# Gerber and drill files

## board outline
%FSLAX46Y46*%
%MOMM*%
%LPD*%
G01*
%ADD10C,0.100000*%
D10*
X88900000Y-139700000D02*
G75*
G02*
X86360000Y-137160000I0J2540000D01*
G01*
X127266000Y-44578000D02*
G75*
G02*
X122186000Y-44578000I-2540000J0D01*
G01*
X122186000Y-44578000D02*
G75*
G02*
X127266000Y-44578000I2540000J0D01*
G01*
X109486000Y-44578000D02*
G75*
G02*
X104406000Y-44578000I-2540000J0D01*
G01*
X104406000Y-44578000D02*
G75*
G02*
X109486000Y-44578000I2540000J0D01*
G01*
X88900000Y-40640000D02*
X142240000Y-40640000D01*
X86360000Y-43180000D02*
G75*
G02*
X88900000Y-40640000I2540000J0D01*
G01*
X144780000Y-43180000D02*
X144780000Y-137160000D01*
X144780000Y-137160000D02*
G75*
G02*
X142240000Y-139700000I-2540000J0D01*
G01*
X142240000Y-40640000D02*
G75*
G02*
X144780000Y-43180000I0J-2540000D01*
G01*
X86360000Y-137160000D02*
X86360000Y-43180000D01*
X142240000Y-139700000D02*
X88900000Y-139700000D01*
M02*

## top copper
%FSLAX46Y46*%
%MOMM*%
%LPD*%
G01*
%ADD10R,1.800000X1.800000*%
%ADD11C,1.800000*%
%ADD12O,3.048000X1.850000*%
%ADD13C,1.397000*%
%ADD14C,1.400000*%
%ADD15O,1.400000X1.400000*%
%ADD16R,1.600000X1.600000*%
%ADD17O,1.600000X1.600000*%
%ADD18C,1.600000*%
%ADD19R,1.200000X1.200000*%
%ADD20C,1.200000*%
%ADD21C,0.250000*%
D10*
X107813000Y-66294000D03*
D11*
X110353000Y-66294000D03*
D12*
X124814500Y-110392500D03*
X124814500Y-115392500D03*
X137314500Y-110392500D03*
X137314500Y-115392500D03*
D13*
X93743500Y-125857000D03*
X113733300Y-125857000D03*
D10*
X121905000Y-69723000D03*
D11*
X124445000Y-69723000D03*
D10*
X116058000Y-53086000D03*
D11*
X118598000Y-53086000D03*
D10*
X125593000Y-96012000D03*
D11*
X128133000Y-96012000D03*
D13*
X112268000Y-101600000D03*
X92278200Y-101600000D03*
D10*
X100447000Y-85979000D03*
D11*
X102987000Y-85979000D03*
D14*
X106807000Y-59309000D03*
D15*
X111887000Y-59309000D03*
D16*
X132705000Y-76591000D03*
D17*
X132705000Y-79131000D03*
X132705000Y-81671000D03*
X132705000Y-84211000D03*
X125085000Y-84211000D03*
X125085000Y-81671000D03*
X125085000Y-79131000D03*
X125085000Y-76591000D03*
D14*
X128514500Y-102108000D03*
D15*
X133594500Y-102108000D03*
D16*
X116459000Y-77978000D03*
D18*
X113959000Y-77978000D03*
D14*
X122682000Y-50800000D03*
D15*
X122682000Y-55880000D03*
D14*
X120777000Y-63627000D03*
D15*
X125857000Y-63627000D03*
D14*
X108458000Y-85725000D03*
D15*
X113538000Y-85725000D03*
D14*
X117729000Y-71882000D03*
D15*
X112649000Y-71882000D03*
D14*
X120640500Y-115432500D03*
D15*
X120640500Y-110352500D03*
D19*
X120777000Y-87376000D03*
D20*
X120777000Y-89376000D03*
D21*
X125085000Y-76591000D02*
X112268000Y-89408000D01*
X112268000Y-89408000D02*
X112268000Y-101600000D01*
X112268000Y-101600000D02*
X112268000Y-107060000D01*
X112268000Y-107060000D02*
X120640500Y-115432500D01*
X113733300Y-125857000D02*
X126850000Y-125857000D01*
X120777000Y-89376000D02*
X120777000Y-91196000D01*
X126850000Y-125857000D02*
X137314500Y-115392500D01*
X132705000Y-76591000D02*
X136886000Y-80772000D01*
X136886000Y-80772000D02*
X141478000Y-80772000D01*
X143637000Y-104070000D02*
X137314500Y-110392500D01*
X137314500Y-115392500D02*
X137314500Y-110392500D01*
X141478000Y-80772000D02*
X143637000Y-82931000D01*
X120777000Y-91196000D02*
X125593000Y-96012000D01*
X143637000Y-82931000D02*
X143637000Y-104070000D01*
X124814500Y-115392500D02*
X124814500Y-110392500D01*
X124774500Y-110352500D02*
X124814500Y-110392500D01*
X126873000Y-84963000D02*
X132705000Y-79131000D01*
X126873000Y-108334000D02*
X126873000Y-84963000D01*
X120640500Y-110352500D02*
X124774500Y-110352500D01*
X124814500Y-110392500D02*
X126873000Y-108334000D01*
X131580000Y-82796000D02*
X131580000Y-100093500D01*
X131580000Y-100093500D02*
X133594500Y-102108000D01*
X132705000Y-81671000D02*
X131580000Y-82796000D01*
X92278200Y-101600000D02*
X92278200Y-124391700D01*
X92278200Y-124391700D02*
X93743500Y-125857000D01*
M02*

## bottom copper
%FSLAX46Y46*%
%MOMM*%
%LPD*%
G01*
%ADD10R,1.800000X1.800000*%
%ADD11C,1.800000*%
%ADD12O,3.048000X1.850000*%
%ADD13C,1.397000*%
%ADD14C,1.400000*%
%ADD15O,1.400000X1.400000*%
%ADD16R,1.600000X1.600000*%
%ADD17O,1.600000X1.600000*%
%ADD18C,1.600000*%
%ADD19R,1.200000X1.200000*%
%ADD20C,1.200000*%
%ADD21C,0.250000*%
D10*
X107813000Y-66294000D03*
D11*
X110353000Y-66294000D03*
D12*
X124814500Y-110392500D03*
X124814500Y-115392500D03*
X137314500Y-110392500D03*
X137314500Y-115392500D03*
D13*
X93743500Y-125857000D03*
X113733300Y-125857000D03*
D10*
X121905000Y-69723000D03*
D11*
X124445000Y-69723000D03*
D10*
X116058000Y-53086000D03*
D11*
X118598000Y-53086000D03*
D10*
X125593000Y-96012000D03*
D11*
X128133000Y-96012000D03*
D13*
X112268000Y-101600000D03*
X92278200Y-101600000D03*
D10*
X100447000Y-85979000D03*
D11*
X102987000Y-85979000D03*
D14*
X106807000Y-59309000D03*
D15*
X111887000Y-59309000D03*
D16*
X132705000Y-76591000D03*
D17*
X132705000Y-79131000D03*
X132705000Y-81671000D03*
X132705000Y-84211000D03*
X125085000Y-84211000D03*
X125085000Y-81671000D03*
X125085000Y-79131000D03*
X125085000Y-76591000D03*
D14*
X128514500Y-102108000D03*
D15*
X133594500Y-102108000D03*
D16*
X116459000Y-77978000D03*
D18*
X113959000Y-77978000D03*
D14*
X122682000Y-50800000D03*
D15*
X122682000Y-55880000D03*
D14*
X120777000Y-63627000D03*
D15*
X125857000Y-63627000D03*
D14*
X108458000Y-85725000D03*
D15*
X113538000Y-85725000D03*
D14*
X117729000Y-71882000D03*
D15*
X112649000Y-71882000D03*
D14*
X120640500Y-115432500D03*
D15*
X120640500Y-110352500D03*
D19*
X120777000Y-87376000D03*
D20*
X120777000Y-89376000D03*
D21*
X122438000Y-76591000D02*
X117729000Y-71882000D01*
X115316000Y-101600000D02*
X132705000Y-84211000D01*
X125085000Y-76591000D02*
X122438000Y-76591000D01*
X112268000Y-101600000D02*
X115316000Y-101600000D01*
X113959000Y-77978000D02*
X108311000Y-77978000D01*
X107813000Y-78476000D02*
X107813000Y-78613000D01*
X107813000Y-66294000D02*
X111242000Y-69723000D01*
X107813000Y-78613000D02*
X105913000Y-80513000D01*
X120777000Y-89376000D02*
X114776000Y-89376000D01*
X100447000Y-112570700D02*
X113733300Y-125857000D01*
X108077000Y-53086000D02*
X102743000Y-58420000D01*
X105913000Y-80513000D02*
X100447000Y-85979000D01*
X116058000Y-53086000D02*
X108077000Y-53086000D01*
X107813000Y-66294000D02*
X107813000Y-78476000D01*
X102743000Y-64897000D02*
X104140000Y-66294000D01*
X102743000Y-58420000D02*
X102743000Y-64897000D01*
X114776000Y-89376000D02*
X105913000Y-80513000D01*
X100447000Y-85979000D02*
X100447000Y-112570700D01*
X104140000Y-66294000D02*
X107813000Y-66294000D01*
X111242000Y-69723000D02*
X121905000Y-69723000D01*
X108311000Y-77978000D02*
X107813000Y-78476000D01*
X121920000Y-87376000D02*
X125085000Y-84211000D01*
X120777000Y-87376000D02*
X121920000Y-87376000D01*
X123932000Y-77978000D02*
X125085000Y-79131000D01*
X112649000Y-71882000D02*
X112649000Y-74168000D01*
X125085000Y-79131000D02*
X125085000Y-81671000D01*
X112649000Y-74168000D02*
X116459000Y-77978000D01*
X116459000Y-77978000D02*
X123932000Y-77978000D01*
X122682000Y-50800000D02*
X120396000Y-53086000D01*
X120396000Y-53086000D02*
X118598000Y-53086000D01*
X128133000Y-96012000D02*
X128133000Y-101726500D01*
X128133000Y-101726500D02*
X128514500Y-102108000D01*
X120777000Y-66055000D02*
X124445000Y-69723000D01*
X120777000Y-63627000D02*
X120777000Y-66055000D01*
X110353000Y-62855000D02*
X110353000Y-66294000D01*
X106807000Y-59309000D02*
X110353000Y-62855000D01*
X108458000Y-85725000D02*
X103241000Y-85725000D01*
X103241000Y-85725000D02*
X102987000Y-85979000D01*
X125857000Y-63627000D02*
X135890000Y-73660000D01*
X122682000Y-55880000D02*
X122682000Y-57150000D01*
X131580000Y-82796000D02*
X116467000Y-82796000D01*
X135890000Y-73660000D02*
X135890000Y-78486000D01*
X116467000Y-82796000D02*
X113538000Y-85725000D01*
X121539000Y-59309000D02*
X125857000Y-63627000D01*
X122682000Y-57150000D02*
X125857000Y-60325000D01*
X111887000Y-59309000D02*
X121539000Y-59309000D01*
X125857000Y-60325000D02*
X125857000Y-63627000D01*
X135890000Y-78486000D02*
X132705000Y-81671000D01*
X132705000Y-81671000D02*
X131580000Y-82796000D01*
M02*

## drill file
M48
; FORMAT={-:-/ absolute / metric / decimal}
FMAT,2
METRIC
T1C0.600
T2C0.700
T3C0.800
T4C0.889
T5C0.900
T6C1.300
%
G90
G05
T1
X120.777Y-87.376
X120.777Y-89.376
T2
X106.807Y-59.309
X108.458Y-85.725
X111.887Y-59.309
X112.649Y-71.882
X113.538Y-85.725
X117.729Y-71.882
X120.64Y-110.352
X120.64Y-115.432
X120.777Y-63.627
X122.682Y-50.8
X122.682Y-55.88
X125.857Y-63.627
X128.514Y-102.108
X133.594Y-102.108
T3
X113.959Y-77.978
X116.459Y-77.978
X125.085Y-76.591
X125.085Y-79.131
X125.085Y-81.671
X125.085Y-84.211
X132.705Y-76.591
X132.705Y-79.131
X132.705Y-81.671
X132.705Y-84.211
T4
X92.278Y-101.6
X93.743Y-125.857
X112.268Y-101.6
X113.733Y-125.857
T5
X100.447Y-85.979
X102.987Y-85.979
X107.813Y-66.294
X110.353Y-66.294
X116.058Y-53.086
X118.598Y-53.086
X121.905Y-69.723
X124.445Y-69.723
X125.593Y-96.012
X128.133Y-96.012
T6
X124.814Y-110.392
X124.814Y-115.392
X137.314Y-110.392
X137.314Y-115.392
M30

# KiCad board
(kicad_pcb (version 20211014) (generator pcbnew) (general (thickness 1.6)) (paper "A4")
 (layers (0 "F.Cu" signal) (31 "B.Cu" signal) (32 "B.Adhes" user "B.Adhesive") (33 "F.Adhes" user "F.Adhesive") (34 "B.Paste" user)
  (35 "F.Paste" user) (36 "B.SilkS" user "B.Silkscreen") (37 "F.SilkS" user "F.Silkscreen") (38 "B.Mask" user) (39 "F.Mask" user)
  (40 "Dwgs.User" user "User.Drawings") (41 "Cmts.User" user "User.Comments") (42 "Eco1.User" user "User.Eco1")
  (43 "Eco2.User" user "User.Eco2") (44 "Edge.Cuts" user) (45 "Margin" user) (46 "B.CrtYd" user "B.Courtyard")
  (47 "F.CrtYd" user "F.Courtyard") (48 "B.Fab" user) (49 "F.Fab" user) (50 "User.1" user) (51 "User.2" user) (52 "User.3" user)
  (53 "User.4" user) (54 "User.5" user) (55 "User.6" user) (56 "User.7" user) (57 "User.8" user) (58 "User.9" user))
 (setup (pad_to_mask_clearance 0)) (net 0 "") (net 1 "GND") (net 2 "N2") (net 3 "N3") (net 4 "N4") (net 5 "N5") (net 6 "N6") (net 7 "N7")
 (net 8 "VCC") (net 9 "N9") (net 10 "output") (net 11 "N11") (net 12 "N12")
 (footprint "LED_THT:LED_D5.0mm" (layer "F.Cu") (at 107.813 66.294)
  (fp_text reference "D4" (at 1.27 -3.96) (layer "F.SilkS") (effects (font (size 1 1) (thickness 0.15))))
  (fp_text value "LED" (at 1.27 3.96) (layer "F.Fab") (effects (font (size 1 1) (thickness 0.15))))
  (pad "1" thru_hole rect (at 0 0) (size 1.8 1.8) (drill 0.9) (layers *.Cu *.Mask) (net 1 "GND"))
  (pad "2" thru_hole circle (at 2.54 0) (size 1.8 1.8) (drill 0.9) (layers *.Cu *.Mask) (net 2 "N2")))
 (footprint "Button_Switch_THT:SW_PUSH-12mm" (layer "F.Cu") (at 124.8145 110.3925)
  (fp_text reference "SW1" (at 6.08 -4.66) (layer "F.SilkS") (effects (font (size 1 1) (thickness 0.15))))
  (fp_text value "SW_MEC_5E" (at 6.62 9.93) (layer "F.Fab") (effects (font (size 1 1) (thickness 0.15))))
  (pad "1" thru_hole oval (at 0 0) (size 3.048 1.85) (drill 1.3) (layers *.Cu *.Mask) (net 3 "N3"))
  (pad "2" thru_hole oval (at 0 5) (size 3.048 1.85) (drill 1.3) (layers *.Cu *.Mask) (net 3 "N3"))
  (pad "3" thru_hole oval (at 12.5 0) (size 3.048 1.85) (drill 1.3) (layers *.Cu *.Mask) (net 1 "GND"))
  (pad "4" thru_hole oval (at 12.5 5) (size 3.048 1.85) (drill 1.3) (layers *.Cu *.Mask) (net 1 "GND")))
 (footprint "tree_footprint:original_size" (layer "F.Cu") (at 117.382022 74.6487)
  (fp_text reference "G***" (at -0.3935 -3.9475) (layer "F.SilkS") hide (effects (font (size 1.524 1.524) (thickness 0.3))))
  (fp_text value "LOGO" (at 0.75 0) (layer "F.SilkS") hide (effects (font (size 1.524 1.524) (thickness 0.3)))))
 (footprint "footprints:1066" (layer "F.Cu") (at 93.7435 125.857)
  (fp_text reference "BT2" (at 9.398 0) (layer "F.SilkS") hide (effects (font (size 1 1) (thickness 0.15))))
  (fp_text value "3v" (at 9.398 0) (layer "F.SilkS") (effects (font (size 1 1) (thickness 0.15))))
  (pad "1" thru_hole circle (at 0 0) (size 1.397 1.397) (drill 0.889) (layers *.Cu *.Mask) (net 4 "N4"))
  (pad "2" thru_hole circle (at 19.9898 0) (size 1.397 1.397) (drill 0.889) (layers *.Cu *.Mask) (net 1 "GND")))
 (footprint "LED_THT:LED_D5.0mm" (layer "F.Cu") (at 121.905 69.723)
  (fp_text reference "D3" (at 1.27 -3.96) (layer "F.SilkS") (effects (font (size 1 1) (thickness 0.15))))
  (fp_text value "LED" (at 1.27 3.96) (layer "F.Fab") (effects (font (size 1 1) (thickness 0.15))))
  (pad "1" thru_hole rect (at 0 0) (size 1.8 1.8) (drill 0.9) (layers *.Cu *.Mask) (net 1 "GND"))
  (pad "2" thru_hole circle (at 2.54 0) (size 1.8 1.8) (drill 0.9) (layers *.Cu *.Mask) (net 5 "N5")))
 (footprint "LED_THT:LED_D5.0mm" (layer "F.Cu") (at 116.058 53.086)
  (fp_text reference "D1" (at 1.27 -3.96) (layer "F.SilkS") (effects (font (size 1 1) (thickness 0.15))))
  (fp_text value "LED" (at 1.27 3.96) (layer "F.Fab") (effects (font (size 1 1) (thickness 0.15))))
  (pad "1" thru_hole rect (at 0 0) (size 1.8 1.8) (drill 0.9) (layers *.Cu *.Mask) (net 1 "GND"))
  (pad "2" thru_hole circle (at 2.54 0) (size 1.8 1.8) (drill 0.9) (layers *.Cu *.Mask) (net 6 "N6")))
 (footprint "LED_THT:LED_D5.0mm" (layer "F.Cu") (at 125.593 96.012)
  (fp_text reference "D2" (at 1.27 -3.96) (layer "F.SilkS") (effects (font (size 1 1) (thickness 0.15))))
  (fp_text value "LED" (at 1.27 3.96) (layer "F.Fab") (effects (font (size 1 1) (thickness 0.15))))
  (pad "1" thru_hole rect (at 0 0) (size 1.8 1.8) (drill 0.9) (layers *.Cu *.Mask) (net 1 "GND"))
  (pad "2" thru_hole circle (at 2.54 0) (size 1.8 1.8) (drill 0.9) (layers *.Cu *.Mask) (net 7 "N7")))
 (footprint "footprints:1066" (layer "F.Cu") (at 112.268 101.6 180)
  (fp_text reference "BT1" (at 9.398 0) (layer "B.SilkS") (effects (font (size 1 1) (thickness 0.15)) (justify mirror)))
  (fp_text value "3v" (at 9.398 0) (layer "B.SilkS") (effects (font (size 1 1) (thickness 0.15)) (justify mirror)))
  (pad "1" thru_hole circle (at 0 0 180) (size 1.397 1.397) (drill 0.889) (layers *.Cu *.Mask) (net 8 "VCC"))
  (pad "2" thru_hole circle (at 19.9898 0 180) (size 1.397 1.397) (drill 0.889) (layers *.Cu *.Mask) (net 4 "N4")))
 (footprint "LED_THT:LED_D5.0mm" (layer "F.Cu") (at 100.447 85.979)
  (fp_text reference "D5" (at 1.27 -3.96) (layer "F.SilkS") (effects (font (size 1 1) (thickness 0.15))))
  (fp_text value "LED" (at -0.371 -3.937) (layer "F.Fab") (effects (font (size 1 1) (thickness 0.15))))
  (pad "1" thru_hole rect (at 0 0) (size 1.8 1.8) (drill 0.9) (layers *.Cu *.Mask) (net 1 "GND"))
  (pad "2" thru_hole circle (at 2.54 0) (size 1.8 1.8) (drill 0.9) (layers *.Cu *.Mask) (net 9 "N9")))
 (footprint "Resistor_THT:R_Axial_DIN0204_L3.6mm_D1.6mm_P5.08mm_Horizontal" (layer "B.Cu") (at 106.807 59.309)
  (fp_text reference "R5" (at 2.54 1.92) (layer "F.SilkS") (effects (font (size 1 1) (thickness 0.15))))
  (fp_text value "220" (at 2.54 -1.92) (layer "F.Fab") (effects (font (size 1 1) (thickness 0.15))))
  (pad "1" thru_hole circle (at 0 0) (size 1.4 1.4) (drill 0.7) (layers *.Cu *.Mask) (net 2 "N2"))
  (pad "2" thru_hole oval (at 5.08 0) (size 1.4 1.4) (drill 0.7) (layers *.Cu *.Mask) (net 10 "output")))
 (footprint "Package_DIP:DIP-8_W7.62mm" (layer "B.Cu") (at 132.705 76.591 180)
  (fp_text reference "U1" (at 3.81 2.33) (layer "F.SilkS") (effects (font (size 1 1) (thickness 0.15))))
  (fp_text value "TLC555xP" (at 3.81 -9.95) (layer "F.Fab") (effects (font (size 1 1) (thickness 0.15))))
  (pad "1" thru_hole rect (at 0 0 180) (size 1.6 1.6) (drill 0.8) (layers *.Cu *.Mask) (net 1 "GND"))
  (pad "2" thru_hole oval (at 0 -2.54 180) (size 1.6 1.6) (drill 0.8) (layers *.Cu *.Mask) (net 3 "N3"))
  (pad "3" thru_hole oval (at 0 -5.08 180) (size 1.6 1.6) (drill 0.8) (layers *.Cu *.Mask) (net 10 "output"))
  (pad "4" thru_hole oval (at 0 -7.62 180) (size 1.6 1.6) (drill 0.8) (layers *.Cu *.Mask) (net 8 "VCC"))
  (pad "5" thru_hole oval (at 7.62 -7.62 180) (size 1.6 1.6) (drill 0.8) (layers *.Cu *.Mask) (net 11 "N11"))
  (pad "6" thru_hole oval (at 7.62 -5.08 180) (size 1.6 1.6) (drill 0.8) (layers *.Cu *.Mask) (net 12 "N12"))
  (pad "7" thru_hole oval (at 7.62 -2.54 180) (size 1.6 1.6) (drill 0.8) (layers *.Cu *.Mask) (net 12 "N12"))
  (pad "8" thru_hole oval (at 7.62 0 180) (size 1.6 1.6) (drill 0.8) (layers *.Cu *.Mask) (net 8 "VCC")))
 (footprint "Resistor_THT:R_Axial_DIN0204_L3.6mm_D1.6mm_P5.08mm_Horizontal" (layer "B.Cu") (at 128.5145 102.108)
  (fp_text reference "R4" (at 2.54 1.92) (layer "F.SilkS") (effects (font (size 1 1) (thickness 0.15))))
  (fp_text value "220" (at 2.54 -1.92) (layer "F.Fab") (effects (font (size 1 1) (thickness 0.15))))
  (pad "1" thru_hole circle (at 0 0) (size 1.4 1.4) (drill 0.7) (layers *.Cu *.Mask) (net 7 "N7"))
  (pad "2" thru_hole oval (at 5.08 0) (size 1.4 1.4) (drill 0.7) (layers *.Cu *.Mask) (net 10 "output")))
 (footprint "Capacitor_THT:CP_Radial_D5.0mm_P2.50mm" (layer "B.Cu") (at 116.459 77.978 180)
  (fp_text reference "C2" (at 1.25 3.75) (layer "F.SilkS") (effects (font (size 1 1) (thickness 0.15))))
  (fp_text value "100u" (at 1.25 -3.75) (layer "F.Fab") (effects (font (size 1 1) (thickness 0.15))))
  (pad "1" thru_hole rect (at 0 0 180) (size 1.6 1.6) (drill 0.8) (layers *.Cu *.Mask) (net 12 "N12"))
  (pad "2" thru_hole circle (at 2.5 0 180) (size 1.6 1.6) (drill 0.8) (layers *.Cu *.Mask) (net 1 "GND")))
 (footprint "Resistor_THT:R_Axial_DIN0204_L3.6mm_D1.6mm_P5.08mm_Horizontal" (layer "B.Cu") (at 122.682 50.8 -90)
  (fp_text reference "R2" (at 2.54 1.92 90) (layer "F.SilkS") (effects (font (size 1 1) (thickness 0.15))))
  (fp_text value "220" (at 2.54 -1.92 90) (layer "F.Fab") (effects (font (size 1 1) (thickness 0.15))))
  (pad "1" thru_hole circle (at 0 0 270) (size 1.4 1.4) (drill 0.7) (layers *.Cu *.Mask) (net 6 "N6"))
  (pad "2" thru_hole oval (at 5.08 0 270) (size 1.4 1.4) (drill 0.7) (layers *.Cu *.Mask) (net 10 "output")))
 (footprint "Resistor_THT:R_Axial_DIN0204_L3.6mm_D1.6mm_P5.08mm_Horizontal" (layer "B.Cu") (at 120.777 63.627)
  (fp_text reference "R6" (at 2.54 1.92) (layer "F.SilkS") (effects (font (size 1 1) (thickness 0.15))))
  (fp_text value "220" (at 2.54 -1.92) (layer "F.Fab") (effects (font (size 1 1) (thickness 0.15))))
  (pad "1" thru_hole circle (at 0 0) (size 1.4 1.4) (drill 0.7) (layers *.Cu *.Mask) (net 5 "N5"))
  (pad "2" thru_hole oval (at 5.08 0) (size 1.4 1.4) (drill 0.7) (layers *.Cu *.Mask) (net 10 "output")))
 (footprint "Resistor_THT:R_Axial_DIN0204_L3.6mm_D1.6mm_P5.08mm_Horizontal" (layer "B.Cu") (at 108.458 85.725)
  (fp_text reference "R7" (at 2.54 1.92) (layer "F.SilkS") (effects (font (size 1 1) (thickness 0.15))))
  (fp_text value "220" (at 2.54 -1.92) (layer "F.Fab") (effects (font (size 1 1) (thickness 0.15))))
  (pad "1" thru_hole circle (at 0 0) (size 1.4 1.4) (drill 0.7) (layers *.Cu *.Mask) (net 9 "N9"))
  (pad "2" thru_hole oval (at 5.08 0) (size 1.4 1.4) (drill 0.7) (layers *.Cu *.Mask) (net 10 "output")))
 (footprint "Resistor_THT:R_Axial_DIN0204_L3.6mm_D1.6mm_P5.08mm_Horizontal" (layer "B.Cu") (at 117.729 71.882 180)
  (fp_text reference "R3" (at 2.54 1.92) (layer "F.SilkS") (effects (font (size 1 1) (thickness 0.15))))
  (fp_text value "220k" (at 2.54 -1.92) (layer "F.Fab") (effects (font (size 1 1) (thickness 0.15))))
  (pad "1" thru_hole circle (at 0 0 180) (size 1.4 1.4) (drill 0.7) (layers *.Cu *.Mask) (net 8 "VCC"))
  (pad "2" thru_hole oval (at 5.08 0 180) (size 1.4 1.4) (drill 0.7) (layers *.Cu *.Mask) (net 12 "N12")))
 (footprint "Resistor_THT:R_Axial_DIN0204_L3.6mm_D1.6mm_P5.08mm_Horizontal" (layer "B.Cu") (at 120.6405 115.4325 90)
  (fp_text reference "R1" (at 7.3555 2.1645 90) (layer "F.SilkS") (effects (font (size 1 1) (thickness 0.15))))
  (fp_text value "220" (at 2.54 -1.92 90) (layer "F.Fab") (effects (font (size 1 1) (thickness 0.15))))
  (pad "1" thru_hole circle (at 0 0 90) (size 1.4 1.4) (drill 0.7) (layers *.Cu *.Mask) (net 8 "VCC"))
  (pad "2" thru_hole oval (at 5.08 0 90) (size 1.4 1.4) (drill 0.7) (layers *.Cu *.Mask) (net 3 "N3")))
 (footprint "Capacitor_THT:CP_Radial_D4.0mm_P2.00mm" (layer "B.Cu") (at 120.777 87.376 -90)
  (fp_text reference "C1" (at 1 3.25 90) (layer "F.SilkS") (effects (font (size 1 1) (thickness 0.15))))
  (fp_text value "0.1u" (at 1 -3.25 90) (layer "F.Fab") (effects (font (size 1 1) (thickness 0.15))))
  (pad "1" thru_hole rect (at 0 0 270) (size 1.2 1.2) (drill 0.6) (layers *.Cu *.Mask) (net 11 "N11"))
  (pad "2" thru_hole circle (at 2 0 270) (size 1.2 1.2) (drill 0.6) (layers *.Cu *.Mask) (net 1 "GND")))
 (gr_arc (start 88.9 139.7) (mid 87.103949 138.956051) (end 86.36 137.16) (layer "Edge.Cuts") (width 0.1))
 (gr_circle (center 124.726 44.578) (end 124.726 42.038) (layer "Edge.Cuts") (width 0.1) (fill none))
 (gr_circle (center 106.946 44.578) (end 106.946 42.038) (layer "Edge.Cuts") (width 0.1) (fill none))
 (gr_line (start 88.9 40.64) (end 142.24 40.64) (layer "Edge.Cuts") (width 0.1))
 (gr_arc (start 86.36 43.18) (mid 87.103949 41.383949) (end 88.9 40.64) (layer "Edge.Cuts") (width 0.1))
 (gr_line (start 144.78 43.18) (end 144.78 137.16) (layer "Edge.Cuts") (width 0.1))
 (gr_arc (start 144.78 137.16) (mid 144.036051 138.956051) (end 142.24 139.7) (layer "Edge.Cuts") (width 0.1))
 (gr_arc (start 142.24 40.64) (mid 144.036051 41.383949) (end 144.78 43.18) (layer "Edge.Cuts") (width 0.1))
 (gr_line (start 86.36 137.16) (end 86.36 43.18) (layer "Edge.Cuts") (width 0.1))
 (gr_line (start 142.24 139.7) (end 88.9 139.7) (layer "Edge.Cuts") (width 0.1))
 (segment (start 125.085 76.591) (end 112.268 89.408) (width 0.25) (layer "F.Cu") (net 8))
 (segment (start 112.268 89.408) (end 112.268 101.6) (width 0.25) (layer "F.Cu") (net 8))
 (segment (start 112.268 101.6) (end 112.268 107.06) (width 0.25) (layer "F.Cu") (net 8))
 (segment (start 112.268 107.06) (end 120.6405 115.4325) (width 0.25) (layer "F.Cu") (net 8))
 (segment (start 122.438 76.591) (end 117.729 71.882) (width 0.25) (layer "B.Cu") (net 8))
 (segment (start 115.316 101.6) (end 132.705 84.211) (width 0.25) (layer "B.Cu") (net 8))
 (segment (start 125.085 76.591) (end 122.438 76.591) (width 0.25) (layer "B.Cu") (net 8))
 (segment (start 112.268 101.6) (end 115.316 101.6) (width 0.25) (layer "B.Cu") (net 8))
 (segment (start 113.7333 125.857) (end 126.85 125.857) (width 0.25) (layer "F.Cu") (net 1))
 (segment (start 120.777 89.376) (end 120.777 91.196) (width 0.25) (layer "F.Cu") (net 1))
 (segment (start 126.85 125.857) (end 137.3145 115.3925) (width 0.25) (layer "F.Cu") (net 1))
 (segment (start 132.705 76.591) (end 136.886 80.772) (width 0.25) (layer "F.Cu") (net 1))
 (segment (start 136.886 80.772) (end 141.478 80.772) (width 0.25) (layer "F.Cu") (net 1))
 (segment (start 143.637 104.07) (end 137.3145 110.3925) (width 0.25) (layer "F.Cu") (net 1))
 (segment (start 137.3145 115.3925) (end 137.3145 110.3925) (width 0.25) (layer "F.Cu") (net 1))
 (segment (start 141.478 80.772) (end 143.637 82.931) (width 0.25) (layer "F.Cu") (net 1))
 (segment (start 120.777 91.196) (end 125.593 96.012) (width 0.25) (layer "F.Cu") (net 1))
 (segment (start 143.637 82.931) (end 143.637 104.07) (width 0.25) (layer "F.Cu") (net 1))
 (segment (start 113.959 77.978) (end 108.311 77.978) (width 0.25) (layer "B.Cu") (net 1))
 (segment (start 107.813 78.476) (end 107.813 78.613) (width 0.25) (layer "B.Cu") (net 1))
 (segment (start 107.813 66.294) (end 111.242 69.723) (width 0.25) (layer "B.Cu") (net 1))
 (segment (start 107.813 78.613) (end 105.913 80.513) (width 0.25) (layer "B.Cu") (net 1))
 (segment (start 120.777 89.376) (end 114.776 89.376) (width 0.25) (layer "B.Cu") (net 1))
 (segment (start 100.447 112.5707) (end 113.7333 125.857) (width 0.25) (layer "B.Cu") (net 1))
 (segment (start 108.077 53.086) (end 102.743 58.42) (width 0.25) (layer "B.Cu") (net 1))
 (segment (start 105.913 80.513) (end 100.447 85.979) (width 0.25) (layer "B.Cu") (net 1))
 (segment (start 116.058 53.086) (end 108.077 53.086) (width 0.25) (layer "B.Cu") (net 1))
 (segment (start 107.813 66.294) (end 107.813 78.476) (width 0.25) (layer "B.Cu") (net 1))
 (segment (start 102.743 64.897) (end 104.14 66.294) (width 0.25) (layer "B.Cu") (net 1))
 (segment (start 102.743 58.42) (end 102.743 64.897) (width 0.25) (layer "B.Cu") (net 1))
 (segment (start 114.776 89.376) (end 105.913 80.513) (width 0.25) (layer "B.Cu") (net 1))
 (segment (start 100.447 85.979) (end 100.447 112.5707) (width 0.25) (layer "B.Cu") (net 1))
 (segment (start 104.14 66.294) (end 107.813 66.294) (width 0.25) (layer "B.Cu") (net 1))
 (segment (start 111.242 69.723) (end 121.905 69.723) (width 0.25) (layer "B.Cu") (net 1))
 (segment (start 108.311 77.978) (end 107.813 78.476) (width 0.25) (layer "B.Cu") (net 1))
 (segment (start 121.92 87.376) (end 125.085 84.211) (width 0.25) (layer "B.Cu") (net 11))
 (segment (start 120.777 87.376) (end 121.92 87.376) (width 0.25) (layer "B.Cu") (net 11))
 (segment (start 123.932 77.978) (end 125.085 79.131) (width 0.25) (layer "B.Cu") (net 12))
 (segment (start 112.649 71.882) (end 112.649 74.168) (width 0.25) (layer "B.Cu") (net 12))
 (segment (start 125.085 79.131) (end 125.085 81.671) (width 0.25) (layer "B.Cu") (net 12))
 (segment (start 112.649 74.168) (end 116.459 77.978) (width 0.25) (layer "B.Cu") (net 12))
 (segment (start 116.459 77.978) (end 123.932 77.978) (width 0.25) (layer "B.Cu") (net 12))
 (segment (start 122.682 50.8) (end 120.396 53.086) (width 0.25) (layer "B.Cu") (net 6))
 (segment (start 120.396 53.086) (end 118.598 53.086) (width 0.25) (layer "B.Cu") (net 6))
 (segment (start 128.133 96.012) (end 128.133 101.7265) (width 0.25) (layer "B.Cu") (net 7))
 (segment (start 128.133 101.7265) (end 128.5145 102.108) (width 0.25) (layer "B.Cu") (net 7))
 (segment (start 120.777 66.055) (end 124.445 69.723) (width 0.25) (layer "B.Cu") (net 5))
 (segment (start 120.777 63.627) (end 120.777 66.055) (width 0.25) (layer "B.Cu") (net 5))
 (segment (start 110.353 62.855) (end 110.353 66.294) (width 0.25) (layer "B.Cu") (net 2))
 (segment (start 106.807 59.309) (end 110.353 62.855) (width 0.25) (layer "B.Cu") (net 2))
 (segment (start 108.458 85.725) (end 103.241 85.725) (width 0.25) (layer "B.Cu") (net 9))
 (segment (start 103.241 85.725) (end 102.987 85.979) (width 0.25) (layer "B.Cu") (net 9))
 (segment (start 124.8145 115.3925) (end 124.8145 110.3925) (width 0.25) (layer "F.Cu") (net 3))
 (segment (start 124.7745 110.3525) (end 124.8145 110.3925) (width 0.25) (layer "F.Cu") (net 3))
 (segment (start 126.873 84.963) (end 132.705 79.131) (width 0.25) (layer "F.Cu") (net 3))
 (segment (start 126.873 108.334) (end 126.873 84.963) (width 0.25) (layer "F.Cu") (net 3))
 (segment (start 120.6405 110.3525) (end 124.7745 110.3525) (width 0.25) (layer "F.Cu") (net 3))
 (segment (start 124.8145 110.3925) (end 126.873 108.334) (width 0.25) (layer "F.Cu") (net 3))
 (segment (start 131.58 82.796) (end 131.58 100.0935) (width 0.25) (layer "F.Cu") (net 10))
 (segment (start 131.58 100.0935) (end 133.5945 102.108) (width 0.25) (layer "F.Cu") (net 10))
 (segment (start 132.705 81.671) (end 131.58 82.796) (width 0.25) (layer "F.Cu") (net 10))
 (segment (start 125.857 63.627) (end 135.89 73.66) (width 0.25) (layer "B.Cu") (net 10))
 (segment (start 122.682 55.88) (end 122.682 57.15) (width 0.25) (layer "B.Cu") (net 10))
 (segment (start 131.58 82.796) (end 116.467 82.796) (width 0.25) (layer "B.Cu") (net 10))
 (segment (start 135.89 73.66) (end 135.89 78.486) (width 0.25) (layer "B.Cu") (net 10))
 (segment (start 116.467 82.796) (end 113.538 85.725) (width 0.25) (layer "B.Cu") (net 10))
 (segment (start 121.539 59.309) (end 125.857 63.627) (width 0.25) (layer "B.Cu") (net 10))
 (segment (start 122.682 57.15) (end 125.857 60.325) (width 0.25) (layer "B.Cu") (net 10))
 (segment (start 111.887 59.309) (end 121.539 59.309) (width 0.25) (layer "B.Cu") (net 10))
 (segment (start 125.857 60.325) (end 125.857 63.627) (width 0.25) (layer "B.Cu") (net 10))
 (segment (start 135.89 78.486) (end 132.705 81.671) (width 0.25) (layer "B.Cu") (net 10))
 (segment (start 132.705 81.671) (end 131.58 82.796) (width 0.25) (layer "B.Cu") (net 10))
 (segment (start 92.2782 101.6) (end 92.2782 124.3917) (width 0.25) (layer "F.Cu") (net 4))
 (segment (start 92.2782 124.3917) (end 93.7435 125.857) (width 0.25) (layer "F.Cu") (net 4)))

